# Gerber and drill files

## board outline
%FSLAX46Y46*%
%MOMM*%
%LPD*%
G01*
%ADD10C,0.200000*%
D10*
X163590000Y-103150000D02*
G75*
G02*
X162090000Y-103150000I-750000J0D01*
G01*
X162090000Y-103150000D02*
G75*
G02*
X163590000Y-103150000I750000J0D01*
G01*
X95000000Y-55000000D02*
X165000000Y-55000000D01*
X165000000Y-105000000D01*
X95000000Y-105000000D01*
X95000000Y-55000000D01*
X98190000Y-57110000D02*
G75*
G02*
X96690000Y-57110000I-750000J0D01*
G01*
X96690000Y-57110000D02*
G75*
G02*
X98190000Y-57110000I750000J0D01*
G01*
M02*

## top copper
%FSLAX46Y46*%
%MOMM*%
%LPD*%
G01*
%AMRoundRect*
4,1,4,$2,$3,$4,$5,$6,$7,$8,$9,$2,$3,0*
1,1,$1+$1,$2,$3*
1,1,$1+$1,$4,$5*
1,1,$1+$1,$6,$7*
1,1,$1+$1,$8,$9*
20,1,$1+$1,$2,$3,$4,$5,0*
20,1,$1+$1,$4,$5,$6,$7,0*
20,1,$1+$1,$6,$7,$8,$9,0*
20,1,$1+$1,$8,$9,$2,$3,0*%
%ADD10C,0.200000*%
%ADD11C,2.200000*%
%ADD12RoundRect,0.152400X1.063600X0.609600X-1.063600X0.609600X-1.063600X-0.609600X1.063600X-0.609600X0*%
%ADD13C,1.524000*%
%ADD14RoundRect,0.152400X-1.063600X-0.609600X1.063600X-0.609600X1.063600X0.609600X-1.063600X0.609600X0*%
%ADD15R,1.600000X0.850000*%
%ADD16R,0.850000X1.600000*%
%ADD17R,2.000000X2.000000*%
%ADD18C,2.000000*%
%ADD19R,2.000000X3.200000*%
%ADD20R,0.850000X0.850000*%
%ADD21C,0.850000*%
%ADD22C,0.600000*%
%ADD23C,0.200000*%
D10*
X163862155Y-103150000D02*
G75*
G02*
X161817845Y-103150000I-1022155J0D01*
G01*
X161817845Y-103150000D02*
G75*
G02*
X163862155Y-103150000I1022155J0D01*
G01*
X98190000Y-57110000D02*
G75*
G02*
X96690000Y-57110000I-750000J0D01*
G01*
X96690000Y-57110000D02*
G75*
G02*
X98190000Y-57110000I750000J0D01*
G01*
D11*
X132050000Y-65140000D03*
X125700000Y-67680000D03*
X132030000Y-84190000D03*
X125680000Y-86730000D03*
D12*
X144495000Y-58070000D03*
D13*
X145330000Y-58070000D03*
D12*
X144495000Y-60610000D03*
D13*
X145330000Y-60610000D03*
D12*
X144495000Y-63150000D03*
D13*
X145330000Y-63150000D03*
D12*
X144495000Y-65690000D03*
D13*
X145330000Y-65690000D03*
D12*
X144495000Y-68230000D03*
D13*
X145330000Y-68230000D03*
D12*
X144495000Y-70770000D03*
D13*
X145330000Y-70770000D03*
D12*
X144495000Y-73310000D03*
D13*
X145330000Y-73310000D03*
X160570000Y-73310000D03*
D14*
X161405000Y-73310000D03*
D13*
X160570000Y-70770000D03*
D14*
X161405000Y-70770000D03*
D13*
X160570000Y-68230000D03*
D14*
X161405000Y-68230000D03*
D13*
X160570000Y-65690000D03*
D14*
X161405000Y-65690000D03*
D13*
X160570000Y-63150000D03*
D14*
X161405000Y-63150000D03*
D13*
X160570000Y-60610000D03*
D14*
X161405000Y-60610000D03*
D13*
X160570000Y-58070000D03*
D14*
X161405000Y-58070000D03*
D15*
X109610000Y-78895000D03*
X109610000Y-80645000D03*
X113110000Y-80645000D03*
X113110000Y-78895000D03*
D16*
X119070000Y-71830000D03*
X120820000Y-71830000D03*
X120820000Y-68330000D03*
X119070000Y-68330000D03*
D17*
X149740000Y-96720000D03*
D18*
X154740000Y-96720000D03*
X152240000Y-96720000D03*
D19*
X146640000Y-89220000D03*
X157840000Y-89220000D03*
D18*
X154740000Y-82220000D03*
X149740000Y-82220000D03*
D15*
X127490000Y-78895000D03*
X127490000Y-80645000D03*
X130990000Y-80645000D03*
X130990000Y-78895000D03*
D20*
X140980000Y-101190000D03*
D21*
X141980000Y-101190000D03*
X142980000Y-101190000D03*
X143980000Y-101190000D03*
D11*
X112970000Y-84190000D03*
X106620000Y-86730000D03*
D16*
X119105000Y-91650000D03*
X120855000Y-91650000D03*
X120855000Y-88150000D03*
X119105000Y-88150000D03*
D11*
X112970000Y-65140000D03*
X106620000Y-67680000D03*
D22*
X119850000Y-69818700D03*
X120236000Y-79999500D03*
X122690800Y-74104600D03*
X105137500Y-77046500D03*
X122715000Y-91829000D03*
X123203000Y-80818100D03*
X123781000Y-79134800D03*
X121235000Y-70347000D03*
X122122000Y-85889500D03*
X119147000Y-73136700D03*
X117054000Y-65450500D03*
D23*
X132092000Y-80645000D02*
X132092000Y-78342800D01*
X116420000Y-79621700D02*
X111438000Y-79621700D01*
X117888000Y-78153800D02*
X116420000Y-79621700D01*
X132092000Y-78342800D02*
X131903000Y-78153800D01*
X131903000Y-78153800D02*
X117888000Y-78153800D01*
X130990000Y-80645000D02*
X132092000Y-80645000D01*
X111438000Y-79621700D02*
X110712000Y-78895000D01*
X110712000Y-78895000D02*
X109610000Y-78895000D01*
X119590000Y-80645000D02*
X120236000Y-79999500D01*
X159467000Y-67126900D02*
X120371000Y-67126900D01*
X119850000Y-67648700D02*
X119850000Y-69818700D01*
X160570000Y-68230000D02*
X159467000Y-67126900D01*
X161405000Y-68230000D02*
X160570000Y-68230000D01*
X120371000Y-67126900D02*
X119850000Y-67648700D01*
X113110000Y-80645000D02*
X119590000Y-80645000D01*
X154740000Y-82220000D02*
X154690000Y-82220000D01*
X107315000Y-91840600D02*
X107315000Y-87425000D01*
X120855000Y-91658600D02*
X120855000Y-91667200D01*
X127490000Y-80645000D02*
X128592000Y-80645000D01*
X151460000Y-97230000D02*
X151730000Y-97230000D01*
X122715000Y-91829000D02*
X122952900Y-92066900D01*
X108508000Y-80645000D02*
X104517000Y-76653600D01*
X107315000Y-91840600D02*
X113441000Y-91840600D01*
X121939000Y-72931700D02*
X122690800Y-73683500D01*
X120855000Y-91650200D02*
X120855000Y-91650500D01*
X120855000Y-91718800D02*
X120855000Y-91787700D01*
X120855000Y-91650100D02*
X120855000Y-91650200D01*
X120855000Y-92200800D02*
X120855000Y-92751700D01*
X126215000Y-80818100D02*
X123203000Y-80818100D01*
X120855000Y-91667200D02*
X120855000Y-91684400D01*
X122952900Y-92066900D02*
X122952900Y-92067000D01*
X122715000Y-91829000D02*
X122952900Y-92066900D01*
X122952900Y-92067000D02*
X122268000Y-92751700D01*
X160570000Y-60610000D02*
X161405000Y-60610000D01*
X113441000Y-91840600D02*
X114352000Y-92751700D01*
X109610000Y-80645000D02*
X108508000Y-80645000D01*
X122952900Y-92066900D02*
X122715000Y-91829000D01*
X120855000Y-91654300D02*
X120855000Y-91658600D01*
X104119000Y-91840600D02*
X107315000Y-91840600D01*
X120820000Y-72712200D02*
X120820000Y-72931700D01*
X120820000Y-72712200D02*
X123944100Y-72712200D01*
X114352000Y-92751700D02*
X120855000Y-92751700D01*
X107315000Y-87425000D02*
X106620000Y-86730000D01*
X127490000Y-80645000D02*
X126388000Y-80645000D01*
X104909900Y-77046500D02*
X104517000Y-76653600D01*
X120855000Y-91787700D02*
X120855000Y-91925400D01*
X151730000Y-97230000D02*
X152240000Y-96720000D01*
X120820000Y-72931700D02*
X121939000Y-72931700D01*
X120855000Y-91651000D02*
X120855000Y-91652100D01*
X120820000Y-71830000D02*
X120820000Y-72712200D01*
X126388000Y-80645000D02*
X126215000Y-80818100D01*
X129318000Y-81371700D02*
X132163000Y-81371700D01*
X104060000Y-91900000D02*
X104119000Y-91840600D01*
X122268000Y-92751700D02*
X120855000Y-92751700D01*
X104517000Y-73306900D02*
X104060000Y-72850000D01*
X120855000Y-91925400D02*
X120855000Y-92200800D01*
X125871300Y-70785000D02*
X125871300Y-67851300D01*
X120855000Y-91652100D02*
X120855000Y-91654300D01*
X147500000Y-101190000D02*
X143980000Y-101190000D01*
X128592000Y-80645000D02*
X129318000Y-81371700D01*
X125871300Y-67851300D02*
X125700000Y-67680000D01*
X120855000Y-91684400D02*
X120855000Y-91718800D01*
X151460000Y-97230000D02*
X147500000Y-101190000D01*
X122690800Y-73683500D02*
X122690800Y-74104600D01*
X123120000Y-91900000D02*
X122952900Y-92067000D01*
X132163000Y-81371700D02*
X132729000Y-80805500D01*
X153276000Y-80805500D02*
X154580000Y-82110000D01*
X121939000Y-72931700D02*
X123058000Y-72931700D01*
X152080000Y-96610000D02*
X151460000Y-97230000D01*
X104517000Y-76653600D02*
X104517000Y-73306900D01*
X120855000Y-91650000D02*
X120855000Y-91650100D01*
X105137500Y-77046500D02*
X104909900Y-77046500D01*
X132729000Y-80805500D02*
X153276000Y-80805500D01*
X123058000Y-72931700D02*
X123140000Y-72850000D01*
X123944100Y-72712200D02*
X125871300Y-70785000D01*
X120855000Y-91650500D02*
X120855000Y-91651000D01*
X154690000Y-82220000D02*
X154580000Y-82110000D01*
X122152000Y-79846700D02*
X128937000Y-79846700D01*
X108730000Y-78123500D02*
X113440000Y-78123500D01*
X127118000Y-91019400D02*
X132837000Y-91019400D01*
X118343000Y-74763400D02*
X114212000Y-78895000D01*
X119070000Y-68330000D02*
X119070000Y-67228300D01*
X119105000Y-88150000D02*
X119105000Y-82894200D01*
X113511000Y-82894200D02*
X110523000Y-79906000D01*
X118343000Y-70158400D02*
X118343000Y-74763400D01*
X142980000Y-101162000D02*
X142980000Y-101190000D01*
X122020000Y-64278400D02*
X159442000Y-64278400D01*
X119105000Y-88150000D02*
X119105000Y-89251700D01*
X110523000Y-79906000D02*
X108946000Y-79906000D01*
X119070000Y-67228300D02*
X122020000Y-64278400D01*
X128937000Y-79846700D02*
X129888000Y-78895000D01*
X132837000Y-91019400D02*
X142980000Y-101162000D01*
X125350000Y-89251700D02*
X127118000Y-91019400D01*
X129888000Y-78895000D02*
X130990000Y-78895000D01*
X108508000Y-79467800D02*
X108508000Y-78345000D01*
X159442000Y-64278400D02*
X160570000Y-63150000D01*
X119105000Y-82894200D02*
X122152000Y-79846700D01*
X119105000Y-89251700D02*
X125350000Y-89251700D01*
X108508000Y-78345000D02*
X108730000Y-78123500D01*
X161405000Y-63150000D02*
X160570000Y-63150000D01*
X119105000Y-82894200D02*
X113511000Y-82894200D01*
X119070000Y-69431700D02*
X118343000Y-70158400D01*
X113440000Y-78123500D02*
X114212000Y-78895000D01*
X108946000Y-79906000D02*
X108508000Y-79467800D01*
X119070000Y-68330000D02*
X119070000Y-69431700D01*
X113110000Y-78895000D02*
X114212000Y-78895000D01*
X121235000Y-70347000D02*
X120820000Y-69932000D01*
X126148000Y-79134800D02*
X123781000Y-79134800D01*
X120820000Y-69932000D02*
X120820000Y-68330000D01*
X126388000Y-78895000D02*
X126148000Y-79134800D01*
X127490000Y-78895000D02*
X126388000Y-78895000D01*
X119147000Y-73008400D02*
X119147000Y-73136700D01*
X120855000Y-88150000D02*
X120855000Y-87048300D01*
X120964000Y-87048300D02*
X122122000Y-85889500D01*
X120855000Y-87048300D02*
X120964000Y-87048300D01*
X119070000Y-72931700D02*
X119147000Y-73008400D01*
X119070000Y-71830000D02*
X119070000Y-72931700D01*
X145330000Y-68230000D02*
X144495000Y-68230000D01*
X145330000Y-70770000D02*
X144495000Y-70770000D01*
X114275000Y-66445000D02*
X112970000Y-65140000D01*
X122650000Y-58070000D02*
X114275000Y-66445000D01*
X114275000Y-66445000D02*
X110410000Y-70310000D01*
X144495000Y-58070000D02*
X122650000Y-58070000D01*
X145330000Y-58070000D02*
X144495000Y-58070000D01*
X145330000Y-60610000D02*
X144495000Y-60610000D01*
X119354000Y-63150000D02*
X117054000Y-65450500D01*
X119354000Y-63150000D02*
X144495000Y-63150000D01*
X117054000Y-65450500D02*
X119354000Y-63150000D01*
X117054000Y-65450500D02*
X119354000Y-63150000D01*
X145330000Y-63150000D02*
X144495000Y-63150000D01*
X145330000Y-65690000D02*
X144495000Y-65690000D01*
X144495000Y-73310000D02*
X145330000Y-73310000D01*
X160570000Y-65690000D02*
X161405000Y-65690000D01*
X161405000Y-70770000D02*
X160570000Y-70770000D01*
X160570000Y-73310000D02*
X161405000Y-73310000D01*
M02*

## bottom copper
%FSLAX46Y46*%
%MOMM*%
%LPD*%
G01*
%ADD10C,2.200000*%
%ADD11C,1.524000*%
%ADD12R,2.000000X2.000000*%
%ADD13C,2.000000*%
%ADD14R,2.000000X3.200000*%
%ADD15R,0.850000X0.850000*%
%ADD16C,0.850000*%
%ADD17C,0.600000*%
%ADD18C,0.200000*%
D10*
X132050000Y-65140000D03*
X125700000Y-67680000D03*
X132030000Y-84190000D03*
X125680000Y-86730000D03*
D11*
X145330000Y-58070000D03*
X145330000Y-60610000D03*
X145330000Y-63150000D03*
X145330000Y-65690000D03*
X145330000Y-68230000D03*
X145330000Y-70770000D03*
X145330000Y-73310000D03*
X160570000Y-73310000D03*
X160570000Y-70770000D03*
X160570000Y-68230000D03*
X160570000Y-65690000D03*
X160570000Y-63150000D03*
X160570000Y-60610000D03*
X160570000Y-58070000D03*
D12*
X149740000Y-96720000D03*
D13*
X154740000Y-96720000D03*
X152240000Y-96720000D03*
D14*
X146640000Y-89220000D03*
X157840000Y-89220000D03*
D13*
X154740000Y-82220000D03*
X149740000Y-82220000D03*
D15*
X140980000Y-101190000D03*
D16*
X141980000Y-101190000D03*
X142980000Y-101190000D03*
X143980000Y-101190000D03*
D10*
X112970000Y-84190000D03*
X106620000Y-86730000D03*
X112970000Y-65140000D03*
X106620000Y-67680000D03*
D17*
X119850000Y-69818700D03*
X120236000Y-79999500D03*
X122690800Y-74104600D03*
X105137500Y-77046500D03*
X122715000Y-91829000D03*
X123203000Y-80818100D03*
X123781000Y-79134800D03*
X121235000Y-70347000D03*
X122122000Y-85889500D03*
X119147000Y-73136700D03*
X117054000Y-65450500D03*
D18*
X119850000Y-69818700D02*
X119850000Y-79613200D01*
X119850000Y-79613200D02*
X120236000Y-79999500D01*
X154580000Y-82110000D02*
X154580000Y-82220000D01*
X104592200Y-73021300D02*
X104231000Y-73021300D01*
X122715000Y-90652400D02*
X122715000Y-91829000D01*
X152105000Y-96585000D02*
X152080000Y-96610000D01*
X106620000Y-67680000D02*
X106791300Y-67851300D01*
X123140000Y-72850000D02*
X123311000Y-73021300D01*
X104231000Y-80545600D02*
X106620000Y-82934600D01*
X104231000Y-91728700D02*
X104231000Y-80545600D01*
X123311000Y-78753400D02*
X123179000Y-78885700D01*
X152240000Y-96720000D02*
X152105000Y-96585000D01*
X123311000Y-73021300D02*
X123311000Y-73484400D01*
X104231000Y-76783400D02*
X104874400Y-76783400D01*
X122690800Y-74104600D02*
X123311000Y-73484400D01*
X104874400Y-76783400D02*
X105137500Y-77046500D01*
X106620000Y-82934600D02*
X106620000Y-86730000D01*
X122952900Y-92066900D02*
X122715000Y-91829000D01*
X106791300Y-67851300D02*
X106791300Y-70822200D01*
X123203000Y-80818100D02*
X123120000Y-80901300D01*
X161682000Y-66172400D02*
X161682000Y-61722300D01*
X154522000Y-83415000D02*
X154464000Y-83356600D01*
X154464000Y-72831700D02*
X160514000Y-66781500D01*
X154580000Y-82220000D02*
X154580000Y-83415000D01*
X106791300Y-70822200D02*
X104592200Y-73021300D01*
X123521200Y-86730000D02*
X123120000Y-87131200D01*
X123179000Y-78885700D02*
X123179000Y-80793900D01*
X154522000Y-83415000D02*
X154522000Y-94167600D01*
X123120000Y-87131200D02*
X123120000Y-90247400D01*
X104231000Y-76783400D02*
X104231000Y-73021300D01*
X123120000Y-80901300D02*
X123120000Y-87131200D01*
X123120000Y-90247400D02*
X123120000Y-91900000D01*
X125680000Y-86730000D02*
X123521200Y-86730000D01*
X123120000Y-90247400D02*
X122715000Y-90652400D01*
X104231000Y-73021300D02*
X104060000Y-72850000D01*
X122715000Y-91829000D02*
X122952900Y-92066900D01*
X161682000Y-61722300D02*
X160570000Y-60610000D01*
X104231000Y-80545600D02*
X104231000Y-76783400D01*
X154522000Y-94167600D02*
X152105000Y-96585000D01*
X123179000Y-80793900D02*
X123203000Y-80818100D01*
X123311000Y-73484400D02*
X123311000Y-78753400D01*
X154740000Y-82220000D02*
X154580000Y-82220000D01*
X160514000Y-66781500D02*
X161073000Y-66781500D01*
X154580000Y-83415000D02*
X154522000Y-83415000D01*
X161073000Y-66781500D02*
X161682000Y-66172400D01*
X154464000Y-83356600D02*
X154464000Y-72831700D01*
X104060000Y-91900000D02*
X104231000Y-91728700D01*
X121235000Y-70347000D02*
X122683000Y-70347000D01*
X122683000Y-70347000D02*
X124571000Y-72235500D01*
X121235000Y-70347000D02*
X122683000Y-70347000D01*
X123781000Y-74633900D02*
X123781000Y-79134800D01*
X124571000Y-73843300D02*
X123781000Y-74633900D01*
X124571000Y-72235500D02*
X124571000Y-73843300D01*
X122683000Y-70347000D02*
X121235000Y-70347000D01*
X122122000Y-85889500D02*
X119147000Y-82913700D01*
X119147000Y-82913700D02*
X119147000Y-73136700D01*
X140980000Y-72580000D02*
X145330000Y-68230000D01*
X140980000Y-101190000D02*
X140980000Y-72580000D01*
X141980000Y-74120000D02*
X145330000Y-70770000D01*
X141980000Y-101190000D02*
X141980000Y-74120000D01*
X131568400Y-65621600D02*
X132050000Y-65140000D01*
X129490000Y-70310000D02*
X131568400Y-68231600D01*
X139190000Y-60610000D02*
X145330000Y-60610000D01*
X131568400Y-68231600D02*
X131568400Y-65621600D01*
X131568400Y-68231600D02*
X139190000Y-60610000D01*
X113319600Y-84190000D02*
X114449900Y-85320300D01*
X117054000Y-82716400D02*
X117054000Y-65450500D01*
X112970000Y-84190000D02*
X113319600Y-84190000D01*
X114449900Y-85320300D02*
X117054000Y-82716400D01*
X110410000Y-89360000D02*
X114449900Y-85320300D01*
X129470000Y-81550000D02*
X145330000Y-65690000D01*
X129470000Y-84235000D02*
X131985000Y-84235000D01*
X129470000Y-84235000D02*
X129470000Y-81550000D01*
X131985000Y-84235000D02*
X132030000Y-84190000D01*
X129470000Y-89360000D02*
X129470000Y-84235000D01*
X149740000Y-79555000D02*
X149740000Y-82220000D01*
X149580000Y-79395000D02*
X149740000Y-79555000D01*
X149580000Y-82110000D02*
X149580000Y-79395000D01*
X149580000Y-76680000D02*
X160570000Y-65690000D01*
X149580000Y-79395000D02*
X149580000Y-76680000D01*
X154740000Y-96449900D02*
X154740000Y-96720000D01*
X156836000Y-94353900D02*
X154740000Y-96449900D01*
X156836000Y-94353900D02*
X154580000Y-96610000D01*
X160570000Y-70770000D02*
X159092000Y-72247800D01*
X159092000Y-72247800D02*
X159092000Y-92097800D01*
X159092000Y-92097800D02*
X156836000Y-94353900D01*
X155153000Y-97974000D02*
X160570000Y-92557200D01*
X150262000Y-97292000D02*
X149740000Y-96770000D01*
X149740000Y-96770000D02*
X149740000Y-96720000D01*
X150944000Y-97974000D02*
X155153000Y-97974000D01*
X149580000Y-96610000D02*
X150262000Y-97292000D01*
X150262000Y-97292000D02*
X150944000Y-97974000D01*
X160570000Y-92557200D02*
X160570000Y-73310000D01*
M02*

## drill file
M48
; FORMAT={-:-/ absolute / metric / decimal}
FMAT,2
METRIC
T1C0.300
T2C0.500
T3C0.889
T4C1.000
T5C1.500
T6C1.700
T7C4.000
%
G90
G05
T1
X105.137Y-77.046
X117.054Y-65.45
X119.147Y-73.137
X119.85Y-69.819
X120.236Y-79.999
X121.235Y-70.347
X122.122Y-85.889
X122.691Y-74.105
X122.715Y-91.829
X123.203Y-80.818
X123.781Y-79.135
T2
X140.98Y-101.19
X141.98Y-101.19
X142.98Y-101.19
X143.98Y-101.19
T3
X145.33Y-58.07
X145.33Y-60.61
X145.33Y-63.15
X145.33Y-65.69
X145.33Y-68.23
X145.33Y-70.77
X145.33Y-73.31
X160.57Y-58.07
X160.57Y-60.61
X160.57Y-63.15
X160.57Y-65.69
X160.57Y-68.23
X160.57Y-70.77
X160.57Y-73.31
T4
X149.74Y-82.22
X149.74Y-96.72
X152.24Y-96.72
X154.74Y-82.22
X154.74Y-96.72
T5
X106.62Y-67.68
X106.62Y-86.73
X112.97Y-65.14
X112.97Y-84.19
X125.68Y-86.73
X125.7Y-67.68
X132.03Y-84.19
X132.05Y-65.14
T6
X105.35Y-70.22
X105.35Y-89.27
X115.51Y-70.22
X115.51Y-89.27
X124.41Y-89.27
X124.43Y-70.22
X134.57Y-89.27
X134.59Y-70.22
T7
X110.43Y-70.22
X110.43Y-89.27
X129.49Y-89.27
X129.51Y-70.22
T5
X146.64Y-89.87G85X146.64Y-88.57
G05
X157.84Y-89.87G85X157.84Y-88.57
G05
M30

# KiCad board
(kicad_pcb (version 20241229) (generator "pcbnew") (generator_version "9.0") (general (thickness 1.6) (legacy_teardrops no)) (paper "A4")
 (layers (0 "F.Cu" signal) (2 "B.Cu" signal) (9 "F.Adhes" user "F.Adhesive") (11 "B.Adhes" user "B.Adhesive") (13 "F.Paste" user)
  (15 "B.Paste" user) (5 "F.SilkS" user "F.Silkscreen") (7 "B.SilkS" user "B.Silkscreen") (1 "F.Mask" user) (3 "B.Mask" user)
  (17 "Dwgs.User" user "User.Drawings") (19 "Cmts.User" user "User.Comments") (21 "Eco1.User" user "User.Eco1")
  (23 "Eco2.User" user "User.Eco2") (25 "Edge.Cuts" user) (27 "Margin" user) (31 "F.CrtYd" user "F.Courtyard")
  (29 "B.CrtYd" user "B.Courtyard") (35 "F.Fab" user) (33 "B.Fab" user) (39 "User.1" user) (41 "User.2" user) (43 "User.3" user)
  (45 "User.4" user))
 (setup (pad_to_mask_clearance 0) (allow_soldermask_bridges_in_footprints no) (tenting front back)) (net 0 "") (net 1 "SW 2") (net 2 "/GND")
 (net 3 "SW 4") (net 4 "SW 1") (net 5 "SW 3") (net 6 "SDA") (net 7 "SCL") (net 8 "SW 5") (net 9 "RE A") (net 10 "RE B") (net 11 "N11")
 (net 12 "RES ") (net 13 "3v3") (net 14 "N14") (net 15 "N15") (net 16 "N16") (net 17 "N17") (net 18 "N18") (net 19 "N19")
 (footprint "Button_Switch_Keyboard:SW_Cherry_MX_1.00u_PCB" (layer "F.Cu") (at 132.05 65.14)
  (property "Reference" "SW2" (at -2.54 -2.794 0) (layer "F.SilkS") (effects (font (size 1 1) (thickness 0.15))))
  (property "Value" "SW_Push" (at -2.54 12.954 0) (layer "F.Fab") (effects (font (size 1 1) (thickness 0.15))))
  (pad "" np_thru_hole circle (at -7.62 5.08) (size 1.7 1.7) (drill 1.7) (layers "*.Cu" "*.Mask"))
  (pad "" np_thru_hole circle (at -2.54 5.08) (size 4 4) (drill 4) (layers "*.Cu" "*.Mask"))
  (pad "" np_thru_hole circle (at 2.54 5.08) (size 1.7 1.7) (drill 1.7) (layers "*.Cu" "*.Mask"))
  (pad "1" thru_hole circle (at 0 0) (size 2.2 2.2) (drill 1.5) (layers "*.Cu" "*.Mask") (remove_unused_layers no) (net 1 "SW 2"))
  (pad "2" thru_hole circle (at -6.35 2.54) (size 2.2 2.2) (drill 1.5) (layers "*.Cu" "*.Mask") (remove_unused_layers no) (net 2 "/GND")))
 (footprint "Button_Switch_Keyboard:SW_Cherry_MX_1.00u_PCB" (layer "F.Cu") (at 132.03 84.19)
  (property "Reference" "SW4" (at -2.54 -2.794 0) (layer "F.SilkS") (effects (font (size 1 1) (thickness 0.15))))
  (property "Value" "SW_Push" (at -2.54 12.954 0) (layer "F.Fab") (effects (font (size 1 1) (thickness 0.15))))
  (pad "" np_thru_hole circle (at -7.62 5.08) (size 1.7 1.7) (drill 1.7) (layers "*.Cu" "*.Mask"))
  (pad "" np_thru_hole circle (at -2.54 5.08) (size 4 4) (drill 4) (layers "*.Cu" "*.Mask"))
  (pad "" np_thru_hole circle (at 2.54 5.08) (size 1.7 1.7) (drill 1.7) (layers "*.Cu" "*.Mask"))
  (pad "1" thru_hole circle (at 0 0) (size 2.2 2.2) (drill 1.5) (layers "*.Cu" "*.Mask") (remove_unused_layers no) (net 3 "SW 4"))
  (pad "2" thru_hole circle (at -6.35 2.54) (size 2.2 2.2) (drill 1.5) (layers "*.Cu" "*.Mask") (remove_unused_layers no) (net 2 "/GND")))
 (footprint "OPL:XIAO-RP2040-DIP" (layer "F.Cu") (at 152.95 65.69)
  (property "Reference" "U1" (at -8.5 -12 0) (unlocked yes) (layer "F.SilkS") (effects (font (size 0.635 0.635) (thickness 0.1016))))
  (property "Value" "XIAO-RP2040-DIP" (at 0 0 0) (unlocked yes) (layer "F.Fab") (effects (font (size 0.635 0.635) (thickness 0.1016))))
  (pad "1" smd roundrect (at -8.455 -7.62 180) (size 2.432 1.524) (layers "F.Cu" "F.Mask") (roundrect_rratio 0.1) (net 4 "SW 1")
   (thermal_bridge_angle 45))
  (pad "1" thru_hole circle (at -7.62 -7.62 180) (size 1.524 1.524) (drill 0.889) (layers "*.Cu" "*.Mask") (remove_unused_layers no)
   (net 4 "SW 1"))
  (pad "2" smd roundrect (at -8.455 -5.08 180) (size 2.432 1.524) (layers "F.Cu" "F.Mask") (roundrect_rratio 0.1) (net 1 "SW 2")
   (thermal_bridge_angle 45))
  (pad "2" thru_hole circle (at -7.62 -5.08 180) (size 1.524 1.524) (drill 0.889) (layers "*.Cu" "*.Mask") (remove_unused_layers no)
   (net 1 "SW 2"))
  (pad "3" smd roundrect (at -8.455 -2.54 180) (size 2.432 1.524) (layers "F.Cu" "F.Mask") (roundrect_rratio 0.1) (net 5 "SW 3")
   (thermal_bridge_angle 45))
  (pad "3" thru_hole circle (at -7.62 -2.54 180) (size 1.524 1.524) (drill 0.889) (layers "*.Cu" "*.Mask") (remove_unused_layers no)
   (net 5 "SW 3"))
  (pad "4" smd roundrect (at -8.455 0 180) (size 2.432 1.524) (layers "F.Cu" "F.Mask") (roundrect_rratio 0.1) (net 3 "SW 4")
   (thermal_bridge_angle 45))
  (pad "4" thru_hole circle (at -7.62 0 180) (size 1.524 1.524) (drill 0.889) (layers "*.Cu" "*.Mask") (remove_unused_layers no)
   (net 3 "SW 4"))
  (pad "5" smd roundrect (at -8.455 2.54 180) (size 2.432 1.524) (layers "F.Cu" "F.Mask") (roundrect_rratio 0.1) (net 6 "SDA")
   (thermal_bridge_angle 45))
  (pad "5" thru_hole circle (at -7.62 2.54 180) (size 1.524 1.524) (drill 0.889) (layers "*.Cu" "*.Mask") (remove_unused_layers no)
   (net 6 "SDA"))
  (pad "6" smd roundrect (at -8.455 5.08 180) (size 2.432 1.524) (layers "F.Cu" "F.Mask") (roundrect_rratio 0.1) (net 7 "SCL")
   (thermal_bridge_angle 45))
  (pad "6" thru_hole circle (at -7.62 5.08 180) (size 1.524 1.524) (drill 0.889) (layers "*.Cu" "*.Mask") (remove_unused_layers no)
   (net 7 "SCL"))
  (pad "7" smd roundrect (at -8.455 7.62 180) (size 2.432 1.524) (layers "F.Cu" "F.Mask") (roundrect_rratio 0.1) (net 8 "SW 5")
   (thermal_bridge_angle 45))
  (pad "7" thru_hole circle (at -7.62 7.62 180) (size 1.524 1.524) (drill 0.889) (layers "*.Cu" "*.Mask") (remove_unused_layers no)
   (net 8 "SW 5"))
  (pad "8" thru_hole circle (at 7.62 7.62) (size 1.524 1.524) (drill 0.889) (layers "*.Cu" "*.Mask") (remove_unused_layers no)
   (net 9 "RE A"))
  (pad "8" smd roundrect (at 8.455 7.62) (size 2.432 1.524) (layers "F.Cu" "F.Mask") (roundrect_rratio 0.1) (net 9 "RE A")
   (thermal_bridge_angle 45))
  (pad "9" thru_hole circle (at 7.62 5.08) (size 1.524 1.524) (drill 0.889) (layers "*.Cu" "*.Mask") (remove_unused_layers no)
   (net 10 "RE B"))
  (pad "9" smd roundrect (at 8.455 5.08) (size 2.432 1.524) (layers "F.Cu" "F.Mask") (roundrect_rratio 0.1) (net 10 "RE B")
   (thermal_bridge_angle 45))
  (pad "10" thru_hole circle (at 7.62 2.54) (size 1.524 1.524) (drill 0.889) (layers "*.Cu" "*.Mask") (remove_unused_layers no)
   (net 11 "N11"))
  (pad "10" smd roundrect (at 8.455 2.54) (size 2.432 1.524) (layers "F.Cu" "F.Mask") (roundrect_rratio 0.1) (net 11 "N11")
   (thermal_bridge_angle 45))
  (pad "11" thru_hole circle (at 7.62 0) (size 1.524 1.524) (drill 0.889) (layers "*.Cu" "*.Mask") (remove_unused_layers no) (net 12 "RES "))
  (pad "11" smd roundrect (at 8.455 0) (size 2.432 1.524) (layers "F.Cu" "F.Mask") (roundrect_rratio 0.1) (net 12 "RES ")
   (thermal_bridge_angle 45))
  (pad "12" thru_hole circle (at 7.62 -2.54) (size 1.524 1.524) (drill 0.889) (layers "*.Cu" "*.Mask") (remove_unused_layers no)
   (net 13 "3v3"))
  (pad "12" smd roundrect (at 8.455 -2.54) (size 2.432 1.524) (layers "F.Cu" "F.Mask") (roundrect_rratio 0.1) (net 13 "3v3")
   (thermal_bridge_angle 45))
  (pad "13" thru_hole circle (at 7.62 -5.08) (size 1.524 1.524) (drill 0.889) (layers "*.Cu" "*.Mask") (remove_unused_layers no)
   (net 2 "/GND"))
  (pad "13" smd roundrect (at 8.455 -5.08) (size 2.432 1.524) (layers "F.Cu" "F.Mask") (roundrect_rratio 0.1) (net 2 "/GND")
   (thermal_bridge_angle 45))
  (pad "14" thru_hole circle (at 7.62 -7.62) (size 1.524 1.524) (drill 0.889) (layers "*.Cu" "*.Mask") (remove_unused_layers no)
   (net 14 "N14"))
  (pad "14" smd roundrect (at 8.455 -7.62) (size 2.432 1.524) (layers "F.Cu" "F.Mask") (roundrect_rratio 0.1) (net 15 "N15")
   (thermal_bridge_angle 45)))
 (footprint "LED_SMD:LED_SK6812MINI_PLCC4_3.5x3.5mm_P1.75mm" (layer "F.Cu") (at 111.36 79.77)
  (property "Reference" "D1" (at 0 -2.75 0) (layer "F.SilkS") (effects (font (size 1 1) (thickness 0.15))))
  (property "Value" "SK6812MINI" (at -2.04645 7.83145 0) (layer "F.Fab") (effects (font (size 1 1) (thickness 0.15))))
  (pad "1" smd rect (at -1.75 -0.875) (size 1.6 0.85) (layers "F.Cu" "F.Mask" "F.Paste") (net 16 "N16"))
  (pad "2" smd rect (at -1.75 0.875) (size 1.6 0.85) (layers "F.Cu" "F.Mask" "F.Paste") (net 2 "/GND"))
  (pad "3" smd rect (at 1.75 0.875) (size 1.6 0.85) (layers "F.Cu" "F.Mask" "F.Paste") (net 11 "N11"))
  (pad "4" smd rect (at 1.75 -0.875) (size 1.6 0.85) (layers "F.Cu" "F.Mask" "F.Paste") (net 13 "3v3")))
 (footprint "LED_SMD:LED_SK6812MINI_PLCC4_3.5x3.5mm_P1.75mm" (layer "F.Cu") (at 119.945 70.08 90)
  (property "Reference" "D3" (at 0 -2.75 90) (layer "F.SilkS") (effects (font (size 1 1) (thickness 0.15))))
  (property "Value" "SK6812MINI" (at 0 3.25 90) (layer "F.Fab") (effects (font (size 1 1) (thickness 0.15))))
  (pad "1" smd rect (at -1.75 -0.875 90) (size 1.6 0.85) (layers "F.Cu" "F.Mask" "F.Paste") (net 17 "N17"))
  (pad "2" smd rect (at -1.75 0.875 90) (size 1.6 0.85) (layers "F.Cu" "F.Mask" "F.Paste") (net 2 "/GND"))
  (pad "3" smd rect (at 1.75 0.875 90) (size 1.6 0.85) (layers "F.Cu" "F.Mask" "F.Paste") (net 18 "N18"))
  (pad "4" smd rect (at 1.75 -0.875 90) (size 1.6 0.85) (layers "F.Cu" "F.Mask" "F.Paste") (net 13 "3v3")))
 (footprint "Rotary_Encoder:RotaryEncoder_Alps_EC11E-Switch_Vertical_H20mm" (layer "F.Cu") (at 149.74 96.72 90)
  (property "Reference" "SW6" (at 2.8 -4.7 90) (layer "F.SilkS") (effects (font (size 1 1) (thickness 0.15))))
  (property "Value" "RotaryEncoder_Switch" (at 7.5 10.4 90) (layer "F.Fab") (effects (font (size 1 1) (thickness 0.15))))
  (pad "A" thru_hole rect (at 0 0 90) (size 2 2) (drill 1) (layers "*.Cu" "*.Mask") (remove_unused_layers no) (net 9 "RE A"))
  (pad "B" thru_hole circle (at 0 5 90) (size 2 2) (drill 1) (layers "*.Cu" "*.Mask") (remove_unused_layers no) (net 10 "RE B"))
  (pad "C" thru_hole circle (at 0 2.5 90) (size 2 2) (drill 1) (layers "*.Cu" "*.Mask") (remove_unused_layers no) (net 2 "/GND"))
  (pad "MP" thru_hole rect (at 7.5 -3.1 90) (size 3.2 2) (drill oval 2.8 1.5) (layers "*.Cu" "*.Mask") (remove_unused_layers no))
  (pad "MP" thru_hole rect (at 7.5 8.1 90) (size 3.2 2) (drill oval 2.8 1.5) (layers "*.Cu" "*.Mask") (remove_unused_layers no))
  (pad "S1" thru_hole circle (at 14.5 5 90) (size 2 2) (drill 1) (layers "*.Cu" "*.Mask") (remove_unused_layers no) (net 2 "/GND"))
  (pad "S2" thru_hole circle (at 14.5 0 90) (size 2 2) (drill 1) (layers "*.Cu" "*.Mask") (remove_unused_layers no) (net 12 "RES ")))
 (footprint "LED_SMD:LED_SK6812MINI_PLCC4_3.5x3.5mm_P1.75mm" (layer "F.Cu") (at 129.24 79.77)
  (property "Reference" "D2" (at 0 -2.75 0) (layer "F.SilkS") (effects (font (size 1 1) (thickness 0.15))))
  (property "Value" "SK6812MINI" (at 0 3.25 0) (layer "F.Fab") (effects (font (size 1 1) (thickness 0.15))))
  (pad "1" smd rect (at -1.75 -0.875) (size 1.6 0.85) (layers "F.Cu" "F.Mask" "F.Paste") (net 18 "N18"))
  (pad "2" smd rect (at -1.75 0.875) (size 1.6 0.85) (layers "F.Cu" "F.Mask" "F.Paste") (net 2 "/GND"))
  (pad "3" smd rect (at 1.75 0.875) (size 1.6 0.85) (layers "F.Cu" "F.Mask" "F.Paste") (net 16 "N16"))
  (pad "4" smd rect (at 1.75 -0.875) (size 1.6 0.85) (layers "F.Cu" "F.Mask" "F.Paste") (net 13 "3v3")))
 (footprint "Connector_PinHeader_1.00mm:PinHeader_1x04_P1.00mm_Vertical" (layer "F.Cu") (at 140.98 101.19 90)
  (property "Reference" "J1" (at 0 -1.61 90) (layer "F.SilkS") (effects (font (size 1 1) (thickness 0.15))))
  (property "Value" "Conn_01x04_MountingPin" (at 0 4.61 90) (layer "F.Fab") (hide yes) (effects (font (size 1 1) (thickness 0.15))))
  (pad "1" thru_hole rect (at 0 0 90) (size 0.85 0.85) (drill 0.5) (layers "*.Cu" "*.Mask") (remove_unused_layers no) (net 6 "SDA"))
  (pad "2" thru_hole circle (at 0 1 90) (size 0.85 0.85) (drill 0.5) (layers "*.Cu" "*.Mask") (remove_unused_layers no) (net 7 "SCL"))
  (pad "3" thru_hole circle (at 0 2 90) (size 0.85 0.85) (drill 0.5) (layers "*.Cu" "*.Mask") (remove_unused_layers no) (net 13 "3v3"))
  (pad "4" thru_hole circle (at 0 3 90) (size 0.85 0.85) (drill 0.5) (layers "*.Cu" "*.Mask") (remove_unused_layers no) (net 2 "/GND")))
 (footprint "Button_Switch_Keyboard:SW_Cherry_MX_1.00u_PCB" (layer "F.Cu") (at 112.97 84.19)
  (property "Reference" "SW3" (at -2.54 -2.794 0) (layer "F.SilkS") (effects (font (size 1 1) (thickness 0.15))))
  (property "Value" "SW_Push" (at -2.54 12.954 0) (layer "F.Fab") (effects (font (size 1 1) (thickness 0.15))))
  (pad "" np_thru_hole circle (at -7.62 5.08) (size 1.7 1.7) (drill 1.7) (layers "*.Cu" "*.Mask"))
  (pad "" np_thru_hole circle (at -2.54 5.08) (size 4 4) (drill 4) (layers "*.Cu" "*.Mask"))
  (pad "" np_thru_hole circle (at 2.54 5.08) (size 1.7 1.7) (drill 1.7) (layers "*.Cu" "*.Mask"))
  (pad "1" thru_hole circle (at 0 0) (size 2.2 2.2) (drill 1.5) (layers "*.Cu" "*.Mask") (remove_unused_layers no) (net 5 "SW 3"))
  (pad "2" thru_hole circle (at -6.35 2.54) (size 2.2 2.2) (drill 1.5) (layers "*.Cu" "*.Mask") (remove_unused_layers no) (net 2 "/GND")))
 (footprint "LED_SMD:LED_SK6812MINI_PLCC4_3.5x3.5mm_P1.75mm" (layer "F.Cu") (at 119.98 89.9 90)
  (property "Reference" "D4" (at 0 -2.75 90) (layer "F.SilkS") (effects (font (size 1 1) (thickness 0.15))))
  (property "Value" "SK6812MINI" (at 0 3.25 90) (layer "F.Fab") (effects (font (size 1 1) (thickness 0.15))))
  (pad "1" smd rect (at -1.75 -0.875 90) (size 1.6 0.85) (layers "F.Cu" "F.Mask" "F.Paste") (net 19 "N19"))
  (pad "2" smd rect (at -1.75 0.875 90) (size 1.6 0.85) (layers "F.Cu" "F.Mask" "F.Paste") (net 2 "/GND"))
  (pad "3" smd rect (at 1.75 0.875 90) (size 1.6 0.85) (layers "F.Cu" "F.Mask" "F.Paste") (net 17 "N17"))
  (pad "4" smd rect (at 1.75 -0.875 90) (size 1.6 0.85) (layers "F.Cu" "F.Mask" "F.Paste") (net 13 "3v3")))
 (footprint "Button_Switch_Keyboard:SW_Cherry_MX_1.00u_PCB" (layer "F.Cu") (at 112.97 65.14)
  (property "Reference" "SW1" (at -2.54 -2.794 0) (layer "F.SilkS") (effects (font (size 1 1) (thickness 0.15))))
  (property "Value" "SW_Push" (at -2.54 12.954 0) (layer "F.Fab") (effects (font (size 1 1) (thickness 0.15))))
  (pad "" np_thru_hole circle (at -7.62 5.08) (size 1.7 1.7) (drill 1.7) (layers "*.Cu" "*.Mask"))
  (pad "" np_thru_hole circle (at -2.54 5.08) (size 4 4) (drill 4) (layers "*.Cu" "*.Mask"))
  (pad "" np_thru_hole circle (at 2.54 5.08) (size 1.7 1.7) (drill 1.7) (layers "*.Cu" "*.Mask"))
  (pad "1" thru_hole circle (at 0 0) (size 2.2 2.2) (drill 1.5) (layers "*.Cu" "*.Mask") (remove_unused_layers no) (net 4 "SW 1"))
  (pad "2" thru_hole circle (at -6.35 2.54) (size 2.2 2.2) (drill 1.5) (layers "*.Cu" "*.Mask") (remove_unused_layers no) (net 2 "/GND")))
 (gr_circle (center 162.84 103.15) (end 163.36 102.27) (stroke (width 0.2) (type default)) (fill no) (layer "F.Cu"))
 (gr_circle (center 97.44 57.11) (end 98.19 57.11) (stroke (width 0.2) (type solid)) (fill no) (layer "F.Cu"))
 (gr_circle (center 162.84 103.15) (end 163.59 103.15) (stroke (width 0.2) (type solid)) (fill no) (layer "Edge.Cuts"))
 (gr_rect (start 95 55) (end 165 105) (stroke (width 0.2) (type solid)) (fill no) (layer "Edge.Cuts"))
 (gr_circle (center 97.44 57.11) (end 98.19 57.11) (stroke (width 0.2) (type solid)) (fill no) (layer "Edge.Cuts"))
 (segment (start 132.092 80.645) (end 132.092 78.3428) (width 0.2) (layer "F.Cu") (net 16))
 (segment (start 116.42 79.6217) (end 111.438 79.6217) (width 0.2) (layer "F.Cu") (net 16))
 (segment (start 117.888 78.1538) (end 116.42 79.6217) (width 0.2) (layer "F.Cu") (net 16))
 (segment (start 132.092 78.3428) (end 131.903 78.1538) (width 0.2) (layer "F.Cu") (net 16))
 (segment (start 131.903 78.1538) (end 117.888 78.1538) (width 0.2) (layer "F.Cu") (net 16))
 (segment (start 130.99 80.645) (end 132.092 80.645) (width 0.2) (layer "F.Cu") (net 16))
 (segment (start 111.438 79.6217) (end 110.712 78.895) (width 0.2) (layer "F.Cu") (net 16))
 (segment (start 110.712 78.895) (end 109.61 78.895) (width 0.2) (layer "F.Cu") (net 16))
 (segment (start 119.59 80.645) (end 120.236 79.9995) (width 0.2) (layer "F.Cu") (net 11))
 (segment (start 159.467 67.1269) (end 120.371 67.1269) (width 0.2) (layer "F.Cu") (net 11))
 (segment (start 119.85 67.6487) (end 119.85 69.8187) (width 0.2) (layer "F.Cu") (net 11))
 (segment (start 160.57 68.23) (end 159.467 67.1269) (width 0.2) (layer "F.Cu") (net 11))
 (segment (start 161.405 68.23) (end 160.57 68.23) (width 0.2) (layer "F.Cu") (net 11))
 (segment (start 120.371 67.1269) (end 119.85 67.6487) (width 0.2) (layer "F.Cu") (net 11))
 (segment (start 113.11 80.645) (end 119.59 80.645) (width 0.2) (layer "F.Cu") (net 11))
 (via (at 119.85 69.8187) (size 0.6) (drill 0.3) (layers "F.Cu" "B.Cu") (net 11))
 (via (at 120.236 79.9995) (size 0.6) (drill 0.3) (layers "F.Cu" "B.Cu") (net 11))
 (segment (start 119.85 69.8187) (end 119.85 79.6132) (width 0.2) (layer "B.Cu") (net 11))
 (segment (start 119.85 79.6132) (end 120.236 79.9995) (width 0.2) (layer "B.Cu") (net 11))
 (segment (start 154.74 82.22) (end 154.69 82.22) (width 0.2) (layer "F.Cu") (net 2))
 (segment (start 107.315 91.8406) (end 107.315 87.425) (width 0.2) (layer "F.Cu") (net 2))
 (segment (start 120.855 91.6586) (end 120.855 91.6672) (width 0.2) (layer "F.Cu") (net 2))
 (segment (start 127.49 80.645) (end 128.592 80.645) (width 0.2) (layer "F.Cu") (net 2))
 (segment (start 151.46 97.23) (end 151.73 97.23) (width 0.2) (layer "F.Cu") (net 2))
 (segment (start 122.715 91.829) (end 122.9529 92.0669) (width 0.2) (layer "F.Cu") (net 2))
 (segment (start 108.508 80.645) (end 104.517 76.6536) (width 0.2) (layer "F.Cu") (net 2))
 (segment (start 107.315 91.8406) (end 113.441 91.8406) (width 0.2) (layer "F.Cu") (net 2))
 (segment (start 121.939 72.9317) (end 122.6908 73.6835) (width 0.2) (layer "F.Cu") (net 2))
 (segment (start 120.855 91.6502) (end 120.855 91.6505) (width 0.2) (layer "F.Cu") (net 2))
 (segment (start 120.855 91.7188) (end 120.855 91.7877) (width 0.2) (layer "F.Cu") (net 2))
 (segment (start 120.855 91.6501) (end 120.855 91.6502) (width 0.2) (layer "F.Cu") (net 2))
 (segment (start 120.855 92.2008) (end 120.855 92.7517) (width 0.2) (layer "F.Cu") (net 2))
 (segment (start 126.215 80.8181) (end 123.203 80.8181) (width 0.2) (layer "F.Cu") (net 2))
 (segment (start 120.855 91.6672) (end 120.855 91.6844) (width 0.2) (layer "F.Cu") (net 2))
 (segment (start 122.9529 92.0669) (end 122.9529 92.067) (width 0.2) (layer "F.Cu") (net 2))
 (segment (start 122.715 91.829) (end 122.9529 92.0669) (width 0.2) (layer "F.Cu") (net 2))
 (segment (start 122.9529 92.067) (end 122.268 92.7517) (width 0.2) (layer "F.Cu") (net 2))
 (segment (start 160.57 60.61) (end 161.405 60.61) (width 0.2) (layer "F.Cu") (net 2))
 (segment (start 113.441 91.8406) (end 114.352 92.7517) (width 0.2) (layer "F.Cu") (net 2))
 (segment (start 109.61 80.645) (end 108.508 80.645) (width 0.2) (layer "F.Cu") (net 2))
 (segment (start 122.9529 92.0669) (end 122.715 91.829) (width 0.2) (layer "F.Cu") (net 2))
 (segment (start 120.855 91.6543) (end 120.855 91.6586) (width 0.2) (layer "F.Cu") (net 2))
 (segment (start 104.119 91.8406) (end 107.315 91.8406) (width 0.2) (layer "F.Cu") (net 2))
 (segment (start 120.82 72.7122) (end 120.82 72.9317) (width 0.2) (layer "F.Cu") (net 2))
 (segment (start 120.82 72.7122) (end 123.9441 72.7122) (width 0.2) (layer "F.Cu") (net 2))
 (segment (start 114.352 92.7517) (end 120.855 92.7517) (width 0.2) (layer "F.Cu") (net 2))
 (segment (start 107.315 87.425) (end 106.62 86.73) (width 0.2) (layer "F.Cu") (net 2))
 (segment (start 127.49 80.645) (end 126.388 80.645) (width 0.2) (layer "F.Cu") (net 2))
 (segment (start 104.9099 77.0465) (end 104.517 76.6536) (width 0.2) (layer "F.Cu") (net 2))
 (segment (start 120.855 91.7877) (end 120.855 91.9254) (width 0.2) (layer "F.Cu") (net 2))
 (segment (start 151.73 97.23) (end 152.24 96.72) (width 0.2) (layer "F.Cu") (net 2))
 (segment (start 120.82 72.9317) (end 121.939 72.9317) (width 0.2) (layer "F.Cu") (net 2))
 (segment (start 120.855 91.651) (end 120.855 91.6521) (width 0.2) (layer "F.Cu") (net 2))
 (segment (start 120.82 71.83) (end 120.82 72.7122) (width 0.2) (layer "F.Cu") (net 2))
 (segment (start 126.388 80.645) (end 126.215 80.8181) (width 0.2) (layer "F.Cu") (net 2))
 (segment (start 129.318 81.3717) (end 132.163 81.3717) (width 0.2) (layer "F.Cu") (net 2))
 (segment (start 104.06 91.9) (end 104.119 91.8406) (width 0.2) (layer "F.Cu") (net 2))
 (segment (start 122.268 92.7517) (end 120.855 92.7517) (width 0.2) (layer "F.Cu") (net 2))
 (segment (start 104.517 73.3069) (end 104.06 72.85) (width 0.2) (layer "F.Cu") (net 2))
 (segment (start 120.855 91.9254) (end 120.855 92.2008) (width 0.2) (layer "F.Cu") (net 2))
 (segment (start 125.8713 70.785) (end 125.8713 67.8513) (width 0.2) (layer "F.Cu") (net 2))
 (segment (start 120.855 91.6521) (end 120.855 91.6543) (width 0.2) (layer "F.Cu") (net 2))
 (segment (start 147.5 101.19) (end 143.98 101.19) (width 0.2) (layer "F.Cu") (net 2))
 (segment (start 128.592 80.645) (end 129.318 81.3717) (width 0.2) (layer "F.Cu") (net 2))
 (segment (start 125.8713 67.8513) (end 125.7 67.68) (width 0.2) (layer "F.Cu") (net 2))
 (segment (start 120.855 91.6844) (end 120.855 91.7188) (width 0.2) (layer "F.Cu") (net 2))
 (segment (start 151.46 97.23) (end 147.5 101.19) (width 0.2) (layer "F.Cu") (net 2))
 (segment (start 122.6908 73.6835) (end 122.6908 74.1046) (width 0.2) (layer "F.Cu") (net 2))
 (segment (start 123.12 91.9) (end 122.9529 92.067) (width 0.2) (layer "F.Cu") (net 2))
 (segment (start 132.163 81.3717) (end 132.729 80.8055) (width 0.2) (layer "F.Cu") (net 2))
 (segment (start 153.276 80.8055) (end 154.58 82.11) (width 0.2) (layer "F.Cu") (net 2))
 (segment (start 121.939 72.9317) (end 123.058 72.9317) (width 0.2) (layer "F.Cu") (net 2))
 (segment (start 152.08 96.61) (end 151.46 97.23) (width 0.2) (layer "F.Cu") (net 2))
 (segment (start 104.517 76.6536) (end 104.517 73.3069) (width 0.2) (layer "F.Cu") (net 2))
 (segment (start 120.855 91.65) (end 120.855 91.6501) (width 0.2) (layer "F.Cu") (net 2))
 (segment (start 105.1375 77.0465) (end 104.9099 77.0465) (width 0.2) (layer "F.Cu") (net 2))
 (segment (start 132.729 80.8055) (end 153.276 80.8055) (width 0.2) (layer "F.Cu") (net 2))
 (segment (start 123.058 72.9317) (end 123.14 72.85) (width 0.2) (layer "F.Cu") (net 2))
 (segment (start 123.9441 72.7122) (end 125.8713 70.785) (width 0.2) (layer "F.Cu") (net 2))
 (segment (start 120.855 91.6505) (end 120.855 91.651) (width 0.2) (layer "F.Cu") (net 2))
 (segment (start 154.69 82.22) (end 154.58 82.11) (width 0.2) (layer "F.Cu") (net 2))
 (via (at 122.6908 74.1046) (size 0.6) (drill 0.3) (layers "F.Cu" "B.Cu") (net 2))
 (via (at 105.1375 77.0465) (size 0.6) (drill 0.3) (layers "F.Cu" "B.Cu") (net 2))
 (via (at 122.715 91.829) (size 0.6) (drill 0.3) (layers "F.Cu" "B.Cu") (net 2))
 (via (at 123.203 80.8181) (size 0.6) (drill 0.3) (layers "F.Cu" "B.Cu") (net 2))
 (segment (start 154.58 82.11) (end 154.58 82.22) (width 0.2) (layer "B.Cu") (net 2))
 (segment (start 104.5922 73.0213) (end 104.231 73.0213) (width 0.2) (layer "B.Cu") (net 2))
 (segment (start 122.715 90.6524) (end 122.715 91.829) (width 0.2) (layer "B.Cu") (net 2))
 (segment (start 152.105 96.585) (end 152.08 96.61) (width 0.2) (layer "B.Cu") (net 2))
 (segment (start 106.62 67.68) (end 106.7913 67.8513) (width 0.2) (layer "B.Cu") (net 2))
 (segment (start 123.14 72.85) (end 123.311 73.0213) (width 0.2) (layer "B.Cu") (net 2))
 (segment (start 104.231 80.5456) (end 106.62 82.9346) (width 0.2) (layer "B.Cu") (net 2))
 (segment (start 104.231 91.7287) (end 104.231 80.5456) (width 0.2) (layer "B.Cu") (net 2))
 (segment (start 123.311 78.7534) (end 123.179 78.8857) (width 0.2) (layer "B.Cu") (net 2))
 (segment (start 152.24 96.72) (end 152.105 96.585) (width 0.2) (layer "B.Cu") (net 2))
 (segment (start 123.311 73.0213) (end 123.311 73.4844) (width 0.2) (layer "B.Cu") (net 2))
 (segment (start 104.231 76.7834) (end 104.8744 76.7834) (width 0.2) (layer "B.Cu") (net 2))
 (segment (start 122.6908 74.1046) (end 123.311 73.4844) (width 0.2) (layer "B.Cu") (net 2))
 (segment (start 104.8744 76.7834) (end 105.1375 77.0465) (width 0.2) (layer "B.Cu") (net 2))
 (segment (start 106.62 82.9346) (end 106.62 86.73) (width 0.2) (layer "B.Cu") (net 2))
 (segment (start 122.9529 92.0669) (end 122.715 91.829) (width 0.2) (layer "B.Cu") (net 2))
 (segment (start 106.7913 67.8513) (end 106.7913 70.8222) (width 0.2) (layer "B.Cu") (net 2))
 (segment (start 123.203 80.8181) (end 123.12 80.9013) (width 0.2) (layer "B.Cu") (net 2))
 (segment (start 161.682 66.1724) (end 161.682 61.7223) (width 0.2) (layer "B.Cu") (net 2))
 (segment (start 154.522 83.415) (end 154.464 83.3566) (width 0.2) (layer "B.Cu") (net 2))
 (segment (start 154.464 72.8317) (end 160.514 66.7815) (width 0.2) (layer "B.Cu") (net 2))
 (segment (start 154.58 82.22) (end 154.58 83.415) (width 0.2) (layer "B.Cu") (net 2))
 (segment (start 106.7913 70.8222) (end 104.5922 73.0213) (width 0.2) (layer "B.Cu") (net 2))
 (segment (start 123.5212 86.73) (end 123.12 87.1312) (width 0.2) (layer "B.Cu") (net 2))
 (segment (start 123.179 78.8857) (end 123.179 80.7939) (width 0.2) (layer "B.Cu") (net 2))
 (segment (start 154.522 83.415) (end 154.522 94.1676) (width 0.2) (layer "B.Cu") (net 2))
 (segment (start 123.12 87.1312) (end 123.12 90.2474) (width 0.2) (layer "B.Cu") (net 2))
 (segment (start 104.231 76.7834) (end 104.231 73.0213) (width 0.2) (layer "B.Cu") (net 2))
 (segment (start 123.12 80.9013) (end 123.12 87.1312) (width 0.2) (layer "B.Cu") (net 2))
 (segment (start 123.12 90.2474) (end 123.12 91.9) (width 0.2) (layer "B.Cu") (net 2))
 (segment (start 125.68 86.73) (end 123.5212 86.73) (width 0.2) (layer "B.Cu") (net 2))
 (segment (start 123.12 90.2474) (end 122.715 90.6524) (width 0.2) (layer "B.Cu") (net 2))
 (segment (start 104.231 73.0213) (end 104.06 72.85) (width 0.2) (layer "B.Cu") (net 2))
 (segment (start 122.715 91.829) (end 122.9529 92.0669) (width 0.2) (layer "B.Cu") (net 2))
 (segment (start 161.682 61.7223) (end 160.57 60.61) (width 0.2) (layer "B.Cu") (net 2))
 (segment (start 104.231 80.5456) (end 104.231 76.7834) (width 0.2) (layer "B.Cu") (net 2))
 (segment (start 154.522 94.1676) (end 152.105 96.585) (width 0.2) (layer "B.Cu") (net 2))
 (segment (start 123.179 80.7939) (end 123.203 80.8181) (width 0.2) (layer "B.Cu") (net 2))
 (segment (start 123.311 73.4844) (end 123.311 78.7534) (width 0.2) (layer "B.Cu") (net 2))
 (segment (start 154.74 82.22) (end 154.58 82.22) (width 0.2) (layer "B.Cu") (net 2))
 (segment (start 160.514 66.7815) (end 161.073 66.7815) (width 0.2) (layer "B.Cu") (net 2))
 (segment (start 154.58 83.415) (end 154.522 83.415) (width 0.2) (layer "B.Cu") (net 2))
 (segment (start 161.073 66.7815) (end 161.682 66.1724) (width 0.2) (layer "B.Cu") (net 2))
 (segment (start 154.464 83.3566) (end 154.464 72.8317) (width 0.2) (layer "B.Cu") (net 2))
 (segment (start 104.06 91.9) (end 104.231 91.7287) (width 0.2) (layer "B.Cu") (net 2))
 (segment (start 122.152 79.8467) (end 128.937 79.8467) (width 0.2) (layer "F.Cu") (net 13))
 (segment (start 108.73 78.1235) (end 113.44 78.1235) (width 0.2) (layer "F.Cu") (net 13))
 (segment (start 127.118 91.0194) (end 132.837 91.0194) (width 0.2) (layer "F.Cu") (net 13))
 (segment (start 118.343 74.7634) (end 114.212 78.895) (width 0.2) (layer "F.Cu") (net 13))
 (segment (start 119.07 68.33) (end 119.07 67.2283) (width 0.2) (layer "F.Cu") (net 13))
 (segment (start 119.105 88.15) (end 119.105 82.8942) (width 0.2) (layer "F.Cu") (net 13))
 (segment (start 113.511 82.8942) (end 110.523 79.906) (width 0.2) (layer "F.Cu") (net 13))
 (segment (start 118.343 70.1584) (end 118.343 74.7634) (width 0.2) (layer "F.Cu") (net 13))
 (segment (start 142.98 101.162) (end 142.98 101.19) (width 0.2) (layer "F.Cu") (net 13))
 (segment (start 122.02 64.2784) (end 159.442 64.2784) (width 0.2) (layer "F.Cu") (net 13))
 (segment (start 119.105 88.15) (end 119.105 89.2517) (width 0.2) (layer "F.Cu") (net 13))
 (segment (start 110.523 79.906) (end 108.946 79.906) (width 0.2) (layer "F.Cu") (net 13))
 (segment (start 119.07 67.2283) (end 122.02 64.2784) (width 0.2) (layer "F.Cu") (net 13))
 (segment (start 128.937 79.8467) (end 129.888 78.895) (width 0.2) (layer "F.Cu") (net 13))
 (segment (start 132.837 91.0194) (end 142.98 101.162) (width 0.2) (layer "F.Cu") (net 13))
 (segment (start 125.35 89.2517) (end 127.118 91.0194) (width 0.2) (layer "F.Cu") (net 13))
 (segment (start 129.888 78.895) (end 130.99 78.895) (width 0.2) (layer "F.Cu") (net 13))
 (segment (start 108.508 79.4678) (end 108.508 78.345) (width 0.2) (layer "F.Cu") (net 13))
 (segment (start 159.442 64.2784) (end 160.57 63.15) (width 0.2) (layer "F.Cu") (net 13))
 (segment (start 119.105 82.8942) (end 122.152 79.8467) (width 0.2) (layer "F.Cu") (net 13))
 (segment (start 119.105 89.2517) (end 125.35 89.2517) (width 0.2) (layer "F.Cu") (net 13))
 (segment (start 108.508 78.345) (end 108.73 78.1235) (width 0.2) (layer "F.Cu") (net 13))
 (segment (start 161.405 63.15) (end 160.57 63.15) (width 0.2) (layer "F.Cu") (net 13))
 (segment (start 119.105 82.8942) (end 113.511 82.8942) (width 0.2) (layer "F.Cu") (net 13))
 (segment (start 119.07 69.4317) (end 118.343 70.1584) (width 0.2) (layer "F.Cu") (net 13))
 (segment (start 113.44 78.1235) (end 114.212 78.895) (width 0.2) (layer "F.Cu") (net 13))
 (segment (start 108.946 79.906) (end 108.508 79.4678) (width 0.2) (layer "F.Cu") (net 13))
 (segment (start 119.07 68.33) (end 119.07 69.4317) (width 0.2) (layer "F.Cu") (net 13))
 (segment (start 113.11 78.895) (end 114.212 78.895) (width 0.2) (layer "F.Cu") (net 13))
 (segment (start 121.235 70.347) (end 120.82 69.932) (width 0.2) (layer "F.Cu") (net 18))
 (segment (start 126.148 79.1348) (end 123.781 79.1348) (width 0.2) (layer "F.Cu") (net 18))
 (segment (start 120.82 69.932) (end 120.82 68.33) (width 0.2) (layer "F.Cu") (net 18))
 (segment (start 126.388 78.895) (end 126.148 79.1348) (width 0.2) (layer "F.Cu") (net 18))
 (segment (start 127.49 78.895) (end 126.388 78.895) (width 0.2) (layer "F.Cu") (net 18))
 (via (at 123.781 79.1348) (size 0.6) (drill 0.3) (layers "F.Cu" "B.Cu") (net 18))
 (via (at 121.235 70.347) (size 0.6) (drill 0.3) (layers "F.Cu" "B.Cu") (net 18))
 (segment (start 121.235 70.347) (end 122.683 70.347) (width 0.2) (layer "B.Cu") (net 18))
 (segment (start 122.683 70.347) (end 124.571 72.2355) (width 0.2) (layer "B.Cu") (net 18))
 (segment (start 121.235 70.347) (end 122.683 70.347) (width 0.2) (layer "B.Cu") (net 18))
 (segment (start 123.781 74.6339) (end 123.781 79.1348) (width 0.2) (layer "B.Cu") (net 18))
 (segment (start 124.571 73.8433) (end 123.781 74.6339) (width 0.2) (layer "B.Cu") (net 18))
 (segment (start 124.571 72.2355) (end 124.571 73.8433) (width 0.2) (layer "B.Cu") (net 18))
 (segment (start 122.683 70.347) (end 121.235 70.347) (width 0.2) (layer "B.Cu") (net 18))
 (segment (start 119.147 73.0084) (end 119.147 73.1367) (width 0.2) (layer "F.Cu") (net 17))
 (segment (start 120.855 88.15) (end 120.855 87.0483) (width 0.2) (layer "F.Cu") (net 17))
 (segment (start 120.964 87.0483) (end 122.122 85.8895) (width 0.2) (layer "F.Cu") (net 17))
 (segment (start 120.855 87.0483) (end 120.964 87.0483) (width 0.2) (layer "F.Cu") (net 17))
 (segment (start 119.07 72.9317) (end 119.147 73.0084) (width 0.2) (layer "F.Cu") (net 17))
 (segment (start 119.07 71.83) (end 119.07 72.9317) (width 0.2) (layer "F.Cu") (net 17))
 (via (at 122.122 85.8895) (size 0.6) (drill 0.3) (layers "F.Cu" "B.Cu") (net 17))
 (via (at 119.147 73.1367) (size 0.6) (drill 0.3) (layers "F.Cu" "B.Cu") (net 17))
 (segment (start 122.122 85.8895) (end 119.147 82.9137) (width 0.2) (layer "B.Cu") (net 17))
 (segment (start 119.147 82.9137) (end 119.147 73.1367) (width 0.2) (layer "B.Cu") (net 17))
 (segment (start 145.33 68.23) (end 144.495 68.23) (width 0.2) (layer "F.Cu") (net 6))
 (segment (start 140.98 72.58) (end 145.33 68.23) (width 0.2) (layer "B.Cu") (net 6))
 (segment (start 140.98 101.19) (end 140.98 72.58) (width 0.2) (layer "B.Cu") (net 6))
 (segment (start 145.33 70.77) (end 144.495 70.77) (width 0.2) (layer "F.Cu") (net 7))
 (segment (start 141.98 74.12) (end 145.33 70.77) (width 0.2) (layer "B.Cu") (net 7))
 (segment (start 141.98 101.19) (end 141.98 74.12) (width 0.2) (layer "B.Cu") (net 7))
 (segment (start 114.275 66.445) (end 112.97 65.14) (width 0.2) (layer "F.Cu") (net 4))
 (segment (start 122.65 58.07) (end 114.275 66.445) (width 0.2) (layer "F.Cu") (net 4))
 (segment (start 114.275 66.445) (end 110.41 70.31) (width 0.2) (layer "F.Cu") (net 4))
 (segment (start 144.495 58.07) (end 122.65 58.07) (width 0.2) (layer "F.Cu") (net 4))
 (segment (start 145.33 58.07) (end 144.495 58.07) (width 0.2) (layer "F.Cu") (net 4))
 (segment (start 145.33 60.61) (end 144.495 60.61) (width 0.2) (layer "F.Cu") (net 1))
 (segment (start 131.5684 65.6216) (end 132.05 65.14) (width 0.2) (layer "B.Cu") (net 1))
 (segment (start 129.49 70.31) (end 131.5684 68.2316) (width 0.2) (layer "B.Cu") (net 1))
 (segment (start 139.19 60.61) (end 145.33 60.61) (width 0.2) (layer "B.Cu") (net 1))
 (segment (start 131.5684 68.2316) (end 131.5684 65.6216) (width 0.2) (layer "B.Cu") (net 1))
 (segment (start 131.5684 68.2316) (end 139.19 60.61) (width 0.2) (layer "B.Cu") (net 1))
 (segment (start 119.354 63.15) (end 117.054 65.4505) (width 0.2) (layer "F.Cu") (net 5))
 (segment (start 119.354 63.15) (end 144.495 63.15) (width 0.2) (layer "F.Cu") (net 5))
 (segment (start 117.054 65.4505) (end 119.354 63.15) (width 0.2) (layer "F.Cu") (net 5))
 (segment (start 117.054 65.4505) (end 119.354 63.15) (width 0.2) (layer "F.Cu") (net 5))
 (segment (start 145.33 63.15) (end 144.495 63.15) (width 0.2) (layer "F.Cu") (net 5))
 (via (at 117.054 65.4505) (size 0.6) (drill 0.3) (layers "F.Cu" "B.Cu") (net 5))
 (segment (start 113.3196 84.19) (end 114.4499 85.3203) (width 0.2) (layer "B.Cu") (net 5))
 (segment (start 117.054 82.7164) (end 117.054 65.4505) (width 0.2) (layer "B.Cu") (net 5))
 (segment (start 112.97 84.19) (end 113.3196 84.19) (width 0.2) (layer "B.Cu") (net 5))
 (segment (start 114.4499 85.3203) (end 117.054 82.7164) (width 0.2) (layer "B.Cu") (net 5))
 (segment (start 110.41 89.36) (end 114.4499 85.3203) (width 0.2) (layer "B.Cu") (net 5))
 (segment (start 145.33 65.69) (end 144.495 65.69) (width 0.2) (layer "F.Cu") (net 3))
 (segment (start 129.47 81.55) (end 145.33 65.69) (width 0.2) (layer "B.Cu") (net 3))
 (segment (start 129.47 84.235) (end 131.985 84.235) (width 0.2) (layer "B.Cu") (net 3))
 (segment (start 129.47 84.235) (end 129.47 81.55) (width 0.2) (layer "B.Cu") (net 3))
 (segment (start 131.985 84.235) (end 132.03 84.19) (width 0.2) (layer "B.Cu") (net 3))
 (segment (start 129.47 89.36) (end 129.47 84.235) (width 0.2) (layer "B.Cu") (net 3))
 (segment (start 144.495 73.31) (end 145.33 73.31) (width 0.2) (layer "F.Cu") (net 8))
 (segment (start 160.57 65.69) (end 161.405 65.69) (width 0.2) (layer "F.Cu") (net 12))
 (segment (start 149.74 79.555) (end 149.74 82.22) (width 0.2) (layer "B.Cu") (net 12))
 (segment (start 149.58 79.395) (end 149.74 79.555) (width 0.2) (layer "B.Cu") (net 12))
 (segment (start 149.58 82.11) (end 149.58 79.395) (width 0.2) (layer "B.Cu") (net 12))
 (segment (start 149.58 76.68) (end 160.57 65.69) (width 0.2) (layer "B.Cu") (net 12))
 (segment (start 149.58 79.395) (end 149.58 76.68) (width 0.2) (layer "B.Cu") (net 12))
 (segment (start 161.405 70.77) (end 160.57 70.77) (width 0.2) (layer "F.Cu") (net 10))
 (segment (start 154.74 96.4499) (end 154.74 96.72) (width 0.2) (layer "B.Cu") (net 10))
 (segment (start 156.836 94.3539) (end 154.74 96.4499) (width 0.2) (layer "B.Cu") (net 10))
 (segment (start 156.836 94.3539) (end 154.58 96.61) (width 0.2) (layer "B.Cu") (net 10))
 (segment (start 160.57 70.77) (end 159.092 72.2478) (width 0.2) (layer "B.Cu") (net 10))
 (segment (start 159.092 72.2478) (end 159.092 92.0978) (width 0.2) (layer "B.Cu") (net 10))
 (segment (start 159.092 92.0978) (end 156.836 94.3539) (width 0.2) (layer "B.Cu") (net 10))
 (segment (start 160.57 73.31) (end 161.405 73.31) (width 0.2) (layer "F.Cu") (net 9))
 (segment (start 155.153 97.974) (end 160.57 92.5572) (width 0.2) (layer "B.Cu") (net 9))
 (segment (start 150.262 97.292) (end 149.74 96.77) (width 0.2) (layer "B.Cu") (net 9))
 (segment (start 149.74 96.77) (end 149.74 96.72) (width 0.2) (layer "B.Cu") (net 9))
 (segment (start 150.944 97.974) (end 155.153 97.974) (width 0.2) (layer "B.Cu") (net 9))
 (segment (start 149.58 96.61) (end 150.262 97.292) (width 0.2) (layer "B.Cu") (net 9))
 (segment (start 150.262 97.292) (end 150.944 97.974) (width 0.2) (layer "B.Cu") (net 9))
 (segment (start 160.57 92.5572) (end 160.57 73.31) (width 0.2) (layer "B.Cu") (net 9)))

